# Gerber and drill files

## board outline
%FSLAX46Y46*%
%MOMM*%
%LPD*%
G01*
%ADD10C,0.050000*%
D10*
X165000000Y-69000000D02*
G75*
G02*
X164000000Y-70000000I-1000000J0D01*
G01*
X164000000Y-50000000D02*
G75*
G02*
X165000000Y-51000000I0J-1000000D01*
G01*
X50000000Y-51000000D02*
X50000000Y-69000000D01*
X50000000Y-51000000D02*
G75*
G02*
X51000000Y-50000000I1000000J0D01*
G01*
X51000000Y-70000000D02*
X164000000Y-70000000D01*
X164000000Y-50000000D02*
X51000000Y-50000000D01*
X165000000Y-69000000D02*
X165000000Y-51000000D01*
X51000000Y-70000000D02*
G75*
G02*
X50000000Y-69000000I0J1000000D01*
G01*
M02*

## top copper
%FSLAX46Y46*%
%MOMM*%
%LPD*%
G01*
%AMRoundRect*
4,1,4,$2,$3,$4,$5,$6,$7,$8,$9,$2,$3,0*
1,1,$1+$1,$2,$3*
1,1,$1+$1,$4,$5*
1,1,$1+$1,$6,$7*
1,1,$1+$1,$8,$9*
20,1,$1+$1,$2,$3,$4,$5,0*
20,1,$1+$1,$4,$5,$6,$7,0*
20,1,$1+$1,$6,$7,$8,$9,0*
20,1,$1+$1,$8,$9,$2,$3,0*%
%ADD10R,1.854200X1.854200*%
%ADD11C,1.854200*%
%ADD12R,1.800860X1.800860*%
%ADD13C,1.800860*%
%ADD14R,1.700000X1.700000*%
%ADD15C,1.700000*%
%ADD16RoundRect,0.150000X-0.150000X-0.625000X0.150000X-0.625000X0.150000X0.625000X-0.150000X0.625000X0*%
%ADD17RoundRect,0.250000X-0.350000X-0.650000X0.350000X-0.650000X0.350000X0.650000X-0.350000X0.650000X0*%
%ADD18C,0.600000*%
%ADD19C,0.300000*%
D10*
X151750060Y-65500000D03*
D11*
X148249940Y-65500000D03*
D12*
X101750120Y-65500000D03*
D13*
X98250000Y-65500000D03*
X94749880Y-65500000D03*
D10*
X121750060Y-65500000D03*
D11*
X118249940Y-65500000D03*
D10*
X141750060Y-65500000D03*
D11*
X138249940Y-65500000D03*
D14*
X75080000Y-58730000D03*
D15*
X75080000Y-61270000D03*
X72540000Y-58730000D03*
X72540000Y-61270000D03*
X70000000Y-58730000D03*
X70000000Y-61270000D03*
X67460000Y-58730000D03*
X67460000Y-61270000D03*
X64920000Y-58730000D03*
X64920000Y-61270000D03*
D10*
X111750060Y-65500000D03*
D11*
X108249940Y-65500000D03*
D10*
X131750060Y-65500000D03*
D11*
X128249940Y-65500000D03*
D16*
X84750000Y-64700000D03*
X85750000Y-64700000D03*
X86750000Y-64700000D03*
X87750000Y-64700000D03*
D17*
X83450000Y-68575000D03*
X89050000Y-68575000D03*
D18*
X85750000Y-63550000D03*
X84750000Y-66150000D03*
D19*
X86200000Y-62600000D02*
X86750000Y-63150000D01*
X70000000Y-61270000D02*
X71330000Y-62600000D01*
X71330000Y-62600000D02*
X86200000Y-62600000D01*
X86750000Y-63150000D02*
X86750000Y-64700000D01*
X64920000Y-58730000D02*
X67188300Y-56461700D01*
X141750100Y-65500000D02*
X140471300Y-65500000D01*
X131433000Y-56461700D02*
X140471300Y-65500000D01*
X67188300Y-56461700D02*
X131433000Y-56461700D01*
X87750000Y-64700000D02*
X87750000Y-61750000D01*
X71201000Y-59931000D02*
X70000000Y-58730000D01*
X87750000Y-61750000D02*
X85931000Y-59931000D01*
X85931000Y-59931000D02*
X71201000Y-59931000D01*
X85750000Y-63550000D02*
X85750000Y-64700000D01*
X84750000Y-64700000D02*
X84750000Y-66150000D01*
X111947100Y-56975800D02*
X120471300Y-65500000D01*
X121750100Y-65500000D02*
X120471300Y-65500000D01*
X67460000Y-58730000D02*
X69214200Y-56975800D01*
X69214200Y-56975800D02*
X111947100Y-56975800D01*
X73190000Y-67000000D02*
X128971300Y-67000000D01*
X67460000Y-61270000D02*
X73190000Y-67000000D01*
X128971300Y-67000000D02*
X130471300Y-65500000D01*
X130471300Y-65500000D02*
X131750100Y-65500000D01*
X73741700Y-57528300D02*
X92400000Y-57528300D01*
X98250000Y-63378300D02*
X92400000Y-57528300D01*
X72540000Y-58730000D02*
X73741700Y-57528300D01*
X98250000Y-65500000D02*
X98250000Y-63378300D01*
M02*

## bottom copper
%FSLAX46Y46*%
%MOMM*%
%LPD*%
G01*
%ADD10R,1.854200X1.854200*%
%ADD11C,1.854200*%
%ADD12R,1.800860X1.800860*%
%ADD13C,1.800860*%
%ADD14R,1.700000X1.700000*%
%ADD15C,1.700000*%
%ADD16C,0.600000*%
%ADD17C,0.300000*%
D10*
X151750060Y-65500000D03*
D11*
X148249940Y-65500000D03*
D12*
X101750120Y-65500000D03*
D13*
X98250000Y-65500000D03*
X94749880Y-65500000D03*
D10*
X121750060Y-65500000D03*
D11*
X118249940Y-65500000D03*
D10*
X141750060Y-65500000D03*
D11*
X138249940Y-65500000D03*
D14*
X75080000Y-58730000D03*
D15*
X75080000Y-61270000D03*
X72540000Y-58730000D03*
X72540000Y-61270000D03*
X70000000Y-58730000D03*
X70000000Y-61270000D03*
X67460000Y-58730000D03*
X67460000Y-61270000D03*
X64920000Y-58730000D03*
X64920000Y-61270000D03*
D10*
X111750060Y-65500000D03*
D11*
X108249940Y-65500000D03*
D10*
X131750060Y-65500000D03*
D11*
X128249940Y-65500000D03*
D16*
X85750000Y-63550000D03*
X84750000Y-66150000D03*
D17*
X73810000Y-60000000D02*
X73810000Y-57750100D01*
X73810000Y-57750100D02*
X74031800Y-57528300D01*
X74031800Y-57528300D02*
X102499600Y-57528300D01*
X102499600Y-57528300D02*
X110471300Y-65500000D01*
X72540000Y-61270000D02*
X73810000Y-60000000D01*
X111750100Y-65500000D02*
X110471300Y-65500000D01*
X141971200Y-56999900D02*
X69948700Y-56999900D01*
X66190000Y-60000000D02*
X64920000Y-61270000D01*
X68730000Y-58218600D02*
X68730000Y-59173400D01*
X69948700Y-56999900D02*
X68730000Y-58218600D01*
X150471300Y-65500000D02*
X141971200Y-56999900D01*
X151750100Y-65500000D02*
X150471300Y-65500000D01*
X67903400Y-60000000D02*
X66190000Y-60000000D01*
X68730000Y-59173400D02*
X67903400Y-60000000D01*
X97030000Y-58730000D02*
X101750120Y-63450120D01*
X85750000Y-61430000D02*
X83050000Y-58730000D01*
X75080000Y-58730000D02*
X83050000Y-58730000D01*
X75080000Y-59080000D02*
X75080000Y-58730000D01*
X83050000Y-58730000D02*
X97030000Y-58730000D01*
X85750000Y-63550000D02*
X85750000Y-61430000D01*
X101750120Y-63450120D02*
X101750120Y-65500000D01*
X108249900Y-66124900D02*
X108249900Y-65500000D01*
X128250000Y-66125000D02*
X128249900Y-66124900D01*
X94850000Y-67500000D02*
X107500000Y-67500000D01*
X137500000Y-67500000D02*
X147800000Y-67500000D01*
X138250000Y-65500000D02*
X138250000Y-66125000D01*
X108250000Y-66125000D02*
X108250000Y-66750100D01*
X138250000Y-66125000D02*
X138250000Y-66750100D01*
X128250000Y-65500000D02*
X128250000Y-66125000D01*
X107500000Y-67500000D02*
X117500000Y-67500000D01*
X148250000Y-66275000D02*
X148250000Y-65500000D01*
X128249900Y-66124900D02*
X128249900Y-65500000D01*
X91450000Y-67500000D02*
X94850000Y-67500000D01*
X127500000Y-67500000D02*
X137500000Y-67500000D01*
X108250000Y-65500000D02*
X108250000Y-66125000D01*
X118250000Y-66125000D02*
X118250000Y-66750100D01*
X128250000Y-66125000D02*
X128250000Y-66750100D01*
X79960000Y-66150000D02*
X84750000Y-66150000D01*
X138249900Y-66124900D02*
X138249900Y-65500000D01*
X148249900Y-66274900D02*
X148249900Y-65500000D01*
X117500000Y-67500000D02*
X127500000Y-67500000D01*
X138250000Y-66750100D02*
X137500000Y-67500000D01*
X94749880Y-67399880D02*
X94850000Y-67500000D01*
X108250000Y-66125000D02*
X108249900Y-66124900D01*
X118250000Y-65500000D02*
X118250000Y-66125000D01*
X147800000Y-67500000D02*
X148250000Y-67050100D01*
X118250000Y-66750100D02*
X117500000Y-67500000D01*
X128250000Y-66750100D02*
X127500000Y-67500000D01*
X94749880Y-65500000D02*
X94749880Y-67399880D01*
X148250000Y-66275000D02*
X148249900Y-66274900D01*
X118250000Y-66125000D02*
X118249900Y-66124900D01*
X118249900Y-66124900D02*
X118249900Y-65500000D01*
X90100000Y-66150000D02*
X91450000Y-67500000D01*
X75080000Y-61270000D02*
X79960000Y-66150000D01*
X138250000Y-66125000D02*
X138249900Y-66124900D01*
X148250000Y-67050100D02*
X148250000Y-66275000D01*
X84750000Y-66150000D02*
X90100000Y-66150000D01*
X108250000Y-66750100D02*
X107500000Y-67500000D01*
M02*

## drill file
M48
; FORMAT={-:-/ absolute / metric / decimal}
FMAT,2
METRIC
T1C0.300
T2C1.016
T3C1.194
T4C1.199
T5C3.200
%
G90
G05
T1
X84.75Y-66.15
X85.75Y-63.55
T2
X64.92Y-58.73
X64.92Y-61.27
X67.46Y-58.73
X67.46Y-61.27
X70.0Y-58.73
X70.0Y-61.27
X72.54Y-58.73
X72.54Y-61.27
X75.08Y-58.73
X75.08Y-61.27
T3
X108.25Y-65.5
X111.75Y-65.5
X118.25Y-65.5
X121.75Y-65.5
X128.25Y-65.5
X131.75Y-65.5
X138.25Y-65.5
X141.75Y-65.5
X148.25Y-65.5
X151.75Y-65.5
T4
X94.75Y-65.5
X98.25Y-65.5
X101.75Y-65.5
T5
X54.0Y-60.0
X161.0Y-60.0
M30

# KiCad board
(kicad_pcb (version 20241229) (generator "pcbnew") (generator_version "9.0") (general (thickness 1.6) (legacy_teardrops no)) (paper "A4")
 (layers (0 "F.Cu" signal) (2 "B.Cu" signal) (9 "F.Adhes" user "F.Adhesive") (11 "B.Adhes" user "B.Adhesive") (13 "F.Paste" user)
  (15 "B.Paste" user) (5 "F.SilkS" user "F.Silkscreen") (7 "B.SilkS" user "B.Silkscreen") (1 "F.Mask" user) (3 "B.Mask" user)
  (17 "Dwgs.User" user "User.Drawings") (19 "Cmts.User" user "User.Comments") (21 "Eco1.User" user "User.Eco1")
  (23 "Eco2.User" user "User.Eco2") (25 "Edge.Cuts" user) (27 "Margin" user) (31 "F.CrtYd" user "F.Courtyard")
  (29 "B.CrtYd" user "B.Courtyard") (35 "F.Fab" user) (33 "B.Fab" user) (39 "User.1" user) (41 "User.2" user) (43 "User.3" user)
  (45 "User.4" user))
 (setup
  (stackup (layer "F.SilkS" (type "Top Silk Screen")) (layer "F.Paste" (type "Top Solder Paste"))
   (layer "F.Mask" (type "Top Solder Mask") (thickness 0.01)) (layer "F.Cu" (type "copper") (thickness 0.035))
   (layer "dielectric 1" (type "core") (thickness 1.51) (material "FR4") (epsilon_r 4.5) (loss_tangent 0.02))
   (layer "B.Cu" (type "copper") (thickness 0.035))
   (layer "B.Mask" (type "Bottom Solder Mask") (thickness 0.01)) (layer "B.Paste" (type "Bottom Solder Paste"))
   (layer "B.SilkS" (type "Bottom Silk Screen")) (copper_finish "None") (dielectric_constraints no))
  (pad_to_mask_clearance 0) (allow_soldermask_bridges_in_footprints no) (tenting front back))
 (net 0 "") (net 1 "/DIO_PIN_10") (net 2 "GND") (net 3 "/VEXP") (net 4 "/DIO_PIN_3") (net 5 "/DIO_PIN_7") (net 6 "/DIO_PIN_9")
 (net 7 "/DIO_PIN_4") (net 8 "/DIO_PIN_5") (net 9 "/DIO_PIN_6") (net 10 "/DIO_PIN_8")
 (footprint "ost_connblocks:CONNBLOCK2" (layer "F.Cu") (at 150 65.5 180)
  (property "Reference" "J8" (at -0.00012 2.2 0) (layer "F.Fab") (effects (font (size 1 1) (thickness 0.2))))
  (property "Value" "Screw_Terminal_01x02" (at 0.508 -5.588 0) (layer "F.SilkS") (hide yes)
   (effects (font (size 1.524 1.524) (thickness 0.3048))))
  (pad "1" thru_hole rect (at -1.75006 0 180) (size 1.8542 1.8542) (drill 1.1938) (layers "*.Cu" "*.Mask") (remove_unused_layers no)
   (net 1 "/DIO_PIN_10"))
  (pad "2" thru_hole circle (at 1.75006 0 180) (size 1.8542 1.8542) (drill 1.1938) (layers "*.Cu" "*.Mask") (remove_unused_layers no)
   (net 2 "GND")))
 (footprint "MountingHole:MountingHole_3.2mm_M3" (layer "F.Cu") (at 54 60)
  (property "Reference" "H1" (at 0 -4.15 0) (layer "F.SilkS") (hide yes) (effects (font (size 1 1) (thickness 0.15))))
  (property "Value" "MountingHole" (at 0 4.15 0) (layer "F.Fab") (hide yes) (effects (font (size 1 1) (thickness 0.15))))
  (pad "" np_thru_hole circle (at 0 0) (size 3.2 3.2) (drill 3.2) (layers "*.Cu" "*.Mask")))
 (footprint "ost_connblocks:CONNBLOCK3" (layer "F.Cu") (at 98.25 65.5 180)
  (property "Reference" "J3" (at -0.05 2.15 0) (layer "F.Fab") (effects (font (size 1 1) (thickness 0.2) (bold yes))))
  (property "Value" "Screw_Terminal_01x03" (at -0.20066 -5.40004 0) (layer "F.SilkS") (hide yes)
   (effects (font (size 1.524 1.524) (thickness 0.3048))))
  (pad "1" thru_hole rect (at -3.50012 0 180) (size 1.80086 1.80086) (drill 1.19888) (layers "*.Cu" "*.Mask") (remove_unused_layers no)
   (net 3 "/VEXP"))
  (pad "2" thru_hole circle (at 0 0 180) (size 1.80086 1.80086) (drill 1.19888) (layers "*.Cu" "*.Mask") (remove_unused_layers no)
   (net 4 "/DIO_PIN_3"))
  (pad "3" thru_hole circle (at 3.50012 0 180) (size 1.80086 1.80086) (drill 1.19888) (layers "*.Cu" "*.Mask") (remove_unused_layers no)
   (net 2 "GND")))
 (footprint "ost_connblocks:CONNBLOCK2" (layer "F.Cu") (at 120 65.5 180)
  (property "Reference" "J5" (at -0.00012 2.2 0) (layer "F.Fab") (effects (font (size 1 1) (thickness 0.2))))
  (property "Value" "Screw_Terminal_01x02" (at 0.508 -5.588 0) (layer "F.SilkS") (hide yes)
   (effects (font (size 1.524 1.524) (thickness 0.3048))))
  (pad "1" thru_hole rect (at -1.75006 0 180) (size 1.8542 1.8542) (drill 1.1938) (layers "*.Cu" "*.Mask") (remove_unused_layers no)
   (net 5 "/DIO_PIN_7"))
  (pad "2" thru_hole circle (at 1.75006 0 180) (size 1.8542 1.8542) (drill 1.1938) (layers "*.Cu" "*.Mask") (remove_unused_layers no)
   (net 2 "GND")))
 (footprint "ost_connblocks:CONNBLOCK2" (layer "F.Cu") (at 140 65.5 180)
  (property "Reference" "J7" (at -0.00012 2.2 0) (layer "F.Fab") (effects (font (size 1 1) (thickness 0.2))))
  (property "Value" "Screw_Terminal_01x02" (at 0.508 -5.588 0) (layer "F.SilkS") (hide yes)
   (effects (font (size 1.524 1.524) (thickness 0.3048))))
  (pad "1" thru_hole rect (at -1.75006 0 180) (size 1.8542 1.8542) (drill 1.1938) (layers "*.Cu" "*.Mask") (remove_unused_layers no)
   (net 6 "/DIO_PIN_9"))
  (pad "2" thru_hole circle (at 1.75006 0 180) (size 1.8542 1.8542) (drill 1.1938) (layers "*.Cu" "*.Mask") (remove_unused_layers no)
   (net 2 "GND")))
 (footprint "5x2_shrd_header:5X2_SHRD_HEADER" (layer "F.Cu") (at 70 60 180)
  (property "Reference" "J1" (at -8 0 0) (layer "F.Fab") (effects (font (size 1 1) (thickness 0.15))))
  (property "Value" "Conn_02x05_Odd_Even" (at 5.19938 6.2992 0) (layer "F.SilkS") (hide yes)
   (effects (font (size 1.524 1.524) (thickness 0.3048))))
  (pad "1" thru_hole rect (at -5.08 1.27 180) (size 1.7 1.7) (drill 1.016) (layers "*.Cu" "*.Mask") (remove_unused_layers no)
   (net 3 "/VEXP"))
  (pad "2" thru_hole circle (at -5.08 -1.27 180) (size 1.7 1.7) (drill 1.016) (layers "*.Cu" "*.Mask") (remove_unused_layers no)
   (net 2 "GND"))
  (pad "3" thru_hole circle (at -2.54 1.27 180) (size 1.7 1.7) (drill 1.016) (layers "*.Cu" "*.Mask") (remove_unused_layers no)
   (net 4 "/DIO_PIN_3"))
  (pad "4" thru_hole circle (at -2.54 -1.27 180) (size 1.7 1.7) (drill 1.016) (layers "*.Cu" "*.Mask") (remove_unused_layers no)
   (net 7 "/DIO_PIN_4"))
  (pad "5" thru_hole circle (at 0 1.27 180) (size 1.7 1.7) (drill 1.016) (layers "*.Cu" "*.Mask") (remove_unused_layers no)
   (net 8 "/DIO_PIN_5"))
  (pad "6" thru_hole circle (at 0 -1.27 180) (size 1.7 1.7) (drill 1.016) (layers "*.Cu" "*.Mask") (remove_unused_layers no)
   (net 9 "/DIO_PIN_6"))
  (pad "7" thru_hole circle (at 2.54 1.27 180) (size 1.7 1.7) (drill 1.016) (layers "*.Cu" "*.Mask") (remove_unused_layers no)
   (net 5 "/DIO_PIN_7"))
  (pad "8" thru_hole circle (at 2.54 -1.27 180) (size 1.7 1.7) (drill 1.016) (layers "*.Cu" "*.Mask") (remove_unused_layers no)
   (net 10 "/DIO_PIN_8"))
  (pad "9" thru_hole circle (at 5.08 1.27 180) (size 1.7 1.7) (drill 1.016) (layers "*.Cu" "*.Mask") (remove_unused_layers no)
   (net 6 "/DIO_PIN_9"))
  (pad "10" thru_hole circle (at 5.08 -1.27 180) (size 1.7 1.7) (drill 1.016) (layers "*.Cu" "*.Mask") (remove_unused_layers no)
   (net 1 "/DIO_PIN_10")))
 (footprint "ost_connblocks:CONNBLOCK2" (layer "F.Cu") (at 110 65.5 180)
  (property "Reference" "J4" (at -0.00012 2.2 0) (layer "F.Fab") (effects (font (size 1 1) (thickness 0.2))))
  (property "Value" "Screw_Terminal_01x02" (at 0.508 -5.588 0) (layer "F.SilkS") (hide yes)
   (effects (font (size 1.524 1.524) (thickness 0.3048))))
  (pad "1" thru_hole rect (at -1.75006 0 180) (size 1.8542 1.8542) (drill 1.1938) (layers "*.Cu" "*.Mask") (remove_unused_layers no)
   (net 7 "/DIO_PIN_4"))
  (pad "2" thru_hole circle (at 1.75006 0 180) (size 1.8542 1.8542) (drill 1.1938) (layers "*.Cu" "*.Mask") (remove_unused_layers no)
   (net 2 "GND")))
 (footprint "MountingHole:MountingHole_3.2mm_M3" (layer "F.Cu") (at 161 60)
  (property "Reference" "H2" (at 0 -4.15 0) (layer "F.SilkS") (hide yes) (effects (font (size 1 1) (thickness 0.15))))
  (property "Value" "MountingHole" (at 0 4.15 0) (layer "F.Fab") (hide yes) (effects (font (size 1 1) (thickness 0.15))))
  (pad "" np_thru_hole circle (at 0 0) (size 3.2 3.2) (drill 3.2) (layers "*.Cu" "*.Mask")))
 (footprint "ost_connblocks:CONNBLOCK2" (layer "F.Cu") (at 130 65.5 180)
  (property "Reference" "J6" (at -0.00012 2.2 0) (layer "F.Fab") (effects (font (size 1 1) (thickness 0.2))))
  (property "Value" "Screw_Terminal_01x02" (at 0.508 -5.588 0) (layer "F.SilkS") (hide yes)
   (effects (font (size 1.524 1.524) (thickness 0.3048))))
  (pad "1" thru_hole rect (at -1.75006 0 180) (size 1.8542 1.8542) (drill 1.1938) (layers "*.Cu" "*.Mask") (remove_unused_layers no)
   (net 10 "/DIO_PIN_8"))
  (pad "2" thru_hole circle (at 1.75006 0 180) (size 1.8542 1.8542) (drill 1.1938) (layers "*.Cu" "*.Mask") (remove_unused_layers no)
   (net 2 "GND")))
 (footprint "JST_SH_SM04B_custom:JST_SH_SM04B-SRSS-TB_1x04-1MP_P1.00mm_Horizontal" (layer "F.Cu") (at 86.25 66.7)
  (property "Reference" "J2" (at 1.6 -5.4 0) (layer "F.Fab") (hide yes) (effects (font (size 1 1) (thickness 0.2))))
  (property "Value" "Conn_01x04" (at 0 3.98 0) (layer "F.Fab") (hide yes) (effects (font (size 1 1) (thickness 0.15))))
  (pad "1" smd roundrect (at -1.5 -2) (size 0.6 1.55) (layers "F.Cu" "F.Mask" "F.Paste") (roundrect_rratio 0.25) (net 2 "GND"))
  (pad "2" smd roundrect (at -0.5 -2) (size 0.6 1.55) (layers "F.Cu" "F.Mask" "F.Paste") (roundrect_rratio 0.25) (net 3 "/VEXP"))
  (pad "3" smd roundrect (at 0.5 -2) (size 0.6 1.55) (layers "F.Cu" "F.Mask" "F.Paste") (roundrect_rratio 0.25) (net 9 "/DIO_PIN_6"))
  (pad "4" smd roundrect (at 1.5 -2) (size 0.6 1.55) (layers "F.Cu" "F.Mask" "F.Paste") (roundrect_rratio 0.25) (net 8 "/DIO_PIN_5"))
  (pad "MP" smd roundrect (at -2.8 1.875) (size 1.2 1.8) (layers "F.Cu" "F.Mask" "F.Paste") (roundrect_rratio 0.208333))
  (pad "MP" smd roundrect (at 2.8 1.875) (size 1.2 1.8) (layers "F.Cu" "F.Mask" "F.Paste") (roundrect_rratio 0.208333)))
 (gr_arc (start 165 69) (mid 164.707107 69.707107) (end 164 70) (stroke (width 0.05) (type default)) (layer "Edge.Cuts"))
 (gr_arc (start 164 50) (mid 164.707107 50.292893) (end 165 51) (stroke (width 0.05) (type default)) (layer "Edge.Cuts"))
 (gr_line (start 50 51) (end 50 69) (stroke (width 0.05) (type default)) (layer "Edge.Cuts"))
 (gr_arc (start 50 51) (mid 50.292893 50.292893) (end 51 50) (stroke (width 0.05) (type default)) (layer "Edge.Cuts"))
 (gr_line (start 51 70) (end 164 70) (stroke (width 0.05) (type default)) (layer "Edge.Cuts"))
 (gr_line (start 164 50) (end 51 50) (stroke (width 0.05) (type default)) (layer "Edge.Cuts"))
 (gr_line (start 165 69) (end 165 51) (stroke (width 0.05) (type default)) (layer "Edge.Cuts"))
 (gr_arc (start 51 70) (mid 50.292893 69.707107) (end 50 69) (stroke (width 0.05) (type default)) (layer "Edge.Cuts"))
 (segment (start 73.81 60) (end 73.81 57.7501) (width 0.3) (layer "B.Cu") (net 7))
 (segment (start 73.81 57.7501) (end 74.0318 57.5283) (width 0.3) (layer "B.Cu") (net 7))
 (segment (start 74.0318 57.5283) (end 102.4996 57.5283) (width 0.3) (layer "B.Cu") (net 7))
 (segment (start 102.4996 57.5283) (end 110.4713 65.5) (width 0.3) (layer "B.Cu") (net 7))
 (segment (start 72.54 61.27) (end 73.81 60) (width 0.3) (layer "B.Cu") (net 7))
 (segment (start 111.7501 65.5) (end 110.4713 65.5) (width 0.3) (layer "B.Cu") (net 7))
 (segment (start 86.2 62.6) (end 86.75 63.15) (width 0.3) (layer "F.Cu") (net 9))
 (segment (start 70 61.27) (end 71.33 62.6) (width 0.3) (layer "F.Cu") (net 9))
 (segment (start 71.33 62.6) (end 86.2 62.6) (width 0.3) (layer "F.Cu") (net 9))
 (segment (start 86.75 63.15) (end 86.75 64.7) (width 0.3) (layer "F.Cu") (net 9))
 (segment (start 64.92 58.73) (end 67.1883 56.4617) (width 0.3) (layer "F.Cu") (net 6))
 (segment (start 141.7501 65.5) (end 140.4713 65.5) (width 0.3) (layer "F.Cu") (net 6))
 (segment (start 131.433 56.4617) (end 140.4713 65.5) (width 0.3) (layer "F.Cu") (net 6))
 (segment (start 67.1883 56.4617) (end 131.433 56.4617) (width 0.3) (layer "F.Cu") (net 6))
 (segment (start 141.9712 56.9999) (end 69.9487 56.9999) (width 0.3) (layer "B.Cu") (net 1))
 (segment (start 66.19 60) (end 64.92 61.27) (width 0.3) (layer "B.Cu") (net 1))
 (segment (start 68.73 58.2186) (end 68.73 59.1734) (width 0.3) (layer "B.Cu") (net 1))
 (segment (start 69.9487 56.9999) (end 68.73 58.2186) (width 0.3) (layer "B.Cu") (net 1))
 (segment (start 150.4713 65.5) (end 141.9712 56.9999) (width 0.3) (layer "B.Cu") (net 1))
 (segment (start 151.7501 65.5) (end 150.4713 65.5) (width 0.3) (layer "B.Cu") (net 1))
 (segment (start 67.9034 60) (end 66.19 60) (width 0.3) (layer "B.Cu") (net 1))
 (segment (start 68.73 59.1734) (end 67.9034 60) (width 0.3) (layer "B.Cu") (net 1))
 (segment (start 87.75 64.7) (end 87.75 61.75) (width 0.3) (layer "F.Cu") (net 8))
 (segment (start 71.201 59.931) (end 70 58.73) (width 0.3) (layer "F.Cu") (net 8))
 (segment (start 87.75 61.75) (end 85.931 59.931) (width 0.3) (layer "F.Cu") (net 8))
 (segment (start 85.931 59.931) (end 71.201 59.931) (width 0.3) (layer "F.Cu") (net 8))
 (segment (start 85.75 63.55) (end 85.75 64.7) (width 0.3) (layer "F.Cu") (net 3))
 (via (at 85.75 63.55) (size 0.6) (drill 0.3) (layers "F.Cu" "B.Cu") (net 3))
 (segment (start 97.03 58.73) (end 101.75012 63.45012) (width 0.3) (layer "B.Cu") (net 3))
 (segment (start 85.75 61.43) (end 83.05 58.73) (width 0.3) (layer "B.Cu") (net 3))
 (segment (start 75.08 58.73) (end 83.05 58.73) (width 0.3) (layer "B.Cu") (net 3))
 (segment (start 75.08 59.08) (end 75.08 58.73) (width 0.3) (layer "B.Cu") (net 3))
 (segment (start 83.05 58.73) (end 97.03 58.73) (width 0.3) (layer "B.Cu") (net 3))
 (segment (start 85.75 63.55) (end 85.75 61.43) (width 0.3) (layer "B.Cu") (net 3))
 (segment (start 101.75012 63.45012) (end 101.75012 65.5) (width 0.3) (layer "B.Cu") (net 3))
 (segment (start 84.75 64.7) (end 84.75 66.15) (width 0.3) (layer "F.Cu") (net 2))
 (via (at 84.75 66.15) (size 0.6) (drill 0.3) (layers "F.Cu" "B.Cu") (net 2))
 (segment (start 108.2499 66.1249) (end 108.2499 65.5) (width 0.3) (layer "B.Cu") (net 2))
 (segment (start 128.25 66.125) (end 128.2499 66.1249) (width 0.3) (layer "B.Cu") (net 2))
 (segment (start 94.85 67.5) (end 107.5 67.5) (width 0.3) (layer "B.Cu") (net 2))
 (segment (start 137.5 67.5) (end 147.8 67.5) (width 0.3) (layer "B.Cu") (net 2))
 (segment (start 138.25 65.5) (end 138.25 66.125) (width 0.3) (layer "B.Cu") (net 2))
 (segment (start 108.25 66.125) (end 108.25 66.7501) (width 0.3) (layer "B.Cu") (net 2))
 (segment (start 138.25 66.125) (end 138.25 66.7501) (width 0.3) (layer "B.Cu") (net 2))
 (segment (start 128.25 65.5) (end 128.25 66.125) (width 0.3) (layer "B.Cu") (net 2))
 (segment (start 107.5 67.5) (end 117.5 67.5) (width 0.3) (layer "B.Cu") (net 2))
 (segment (start 148.25 66.275) (end 148.25 65.5) (width 0.3) (layer "B.Cu") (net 2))
 (segment (start 128.2499 66.1249) (end 128.2499 65.5) (width 0.3) (layer "B.Cu") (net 2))
 (segment (start 91.45 67.5) (end 94.85 67.5) (width 0.3) (layer "B.Cu") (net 2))
 (segment (start 127.5 67.5) (end 137.5 67.5) (width 0.3) (layer "B.Cu") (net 2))
 (segment (start 108.25 65.5) (end 108.25 66.125) (width 0.3) (layer "B.Cu") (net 2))
 (segment (start 118.25 66.125) (end 118.25 66.7501) (width 0.3) (layer "B.Cu") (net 2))
 (segment (start 128.25 66.125) (end 128.25 66.7501) (width 0.3) (layer "B.Cu") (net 2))
 (segment (start 79.96 66.15) (end 84.75 66.15) (width 0.3) (layer "B.Cu") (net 2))
 (segment (start 138.2499 66.1249) (end 138.2499 65.5) (width 0.3) (layer "B.Cu") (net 2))
 (segment (start 148.2499 66.2749) (end 148.2499 65.5) (width 0.3) (layer "B.Cu") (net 2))
 (segment (start 117.5 67.5) (end 127.5 67.5) (width 0.3) (layer "B.Cu") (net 2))
 (segment (start 138.25 66.7501) (end 137.5 67.5) (width 0.3) (layer "B.Cu") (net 2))
 (segment (start 94.74988 67.39988) (end 94.85 67.5) (width 0.3) (layer "B.Cu") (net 2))
 (segment (start 108.25 66.125) (end 108.2499 66.1249) (width 0.3) (layer "B.Cu") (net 2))
 (segment (start 118.25 65.5) (end 118.25 66.125) (width 0.3) (layer "B.Cu") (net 2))
 (segment (start 147.8 67.5) (end 148.25 67.0501) (width 0.3) (layer "B.Cu") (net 2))
 (segment (start 118.25 66.7501) (end 117.5 67.5) (width 0.3) (layer "B.Cu") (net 2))
 (segment (start 128.25 66.7501) (end 127.5 67.5) (width 0.3) (layer "B.Cu") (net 2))
 (segment (start 94.74988 65.5) (end 94.74988 67.39988) (width 0.3) (layer "B.Cu") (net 2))
 (segment (start 148.25 66.275) (end 148.2499 66.2749) (width 0.3) (layer "B.Cu") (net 2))
 (segment (start 118.25 66.125) (end 118.2499 66.1249) (width 0.3) (layer "B.Cu") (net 2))
 (segment (start 118.2499 66.1249) (end 118.2499 65.5) (width 0.3) (layer "B.Cu") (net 2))
 (segment (start 90.1 66.15) (end 91.45 67.5) (width 0.3) (layer "B.Cu") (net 2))
 (segment (start 75.08 61.27) (end 79.96 66.15) (width 0.3) (layer "B.Cu") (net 2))
 (segment (start 138.25 66.125) (end 138.2499 66.1249) (width 0.3) (layer "B.Cu") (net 2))
 (segment (start 148.25 67.0501) (end 148.25 66.275) (width 0.3) (layer "B.Cu") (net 2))
 (segment (start 84.75 66.15) (end 90.1 66.15) (width 0.3) (layer "B.Cu") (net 2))
 (segment (start 108.25 66.7501) (end 107.5 67.5) (width 0.3) (layer "B.Cu") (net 2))
 (segment (start 111.9471 56.9758) (end 120.4713 65.5) (width 0.3) (layer "F.Cu") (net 5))
 (segment (start 121.7501 65.5) (end 120.4713 65.5) (width 0.3) (layer "F.Cu") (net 5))
 (segment (start 67.46 58.73) (end 69.2142 56.9758) (width 0.3) (layer "F.Cu") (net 5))
 (segment (start 69.2142 56.9758) (end 111.9471 56.9758) (width 0.3) (layer "F.Cu") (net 5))
 (segment (start 73.19 67) (end 128.9713 67) (width 0.3) (layer "F.Cu") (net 10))
 (segment (start 67.46 61.27) (end 73.19 67) (width 0.3) (layer "F.Cu") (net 10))
 (segment (start 128.9713 67) (end 130.4713 65.5) (width 0.3) (layer "F.Cu") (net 10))
 (segment (start 130.4713 65.5) (end 131.7501 65.5) (width 0.3) (layer "F.Cu") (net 10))
 (segment (start 73.7417 57.5283) (end 92.4 57.5283) (width 0.3) (layer "F.Cu") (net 4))
 (segment (start 98.25 63.3783) (end 92.4 57.5283) (width 0.3) (layer "F.Cu") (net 4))
 (segment (start 72.54 58.73) (end 73.7417 57.5283) (width 0.3) (layer "F.Cu") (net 4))
 (segment (start 98.25 65.5) (end 98.25 63.3783) (width 0.3) (layer "F.Cu") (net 4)))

